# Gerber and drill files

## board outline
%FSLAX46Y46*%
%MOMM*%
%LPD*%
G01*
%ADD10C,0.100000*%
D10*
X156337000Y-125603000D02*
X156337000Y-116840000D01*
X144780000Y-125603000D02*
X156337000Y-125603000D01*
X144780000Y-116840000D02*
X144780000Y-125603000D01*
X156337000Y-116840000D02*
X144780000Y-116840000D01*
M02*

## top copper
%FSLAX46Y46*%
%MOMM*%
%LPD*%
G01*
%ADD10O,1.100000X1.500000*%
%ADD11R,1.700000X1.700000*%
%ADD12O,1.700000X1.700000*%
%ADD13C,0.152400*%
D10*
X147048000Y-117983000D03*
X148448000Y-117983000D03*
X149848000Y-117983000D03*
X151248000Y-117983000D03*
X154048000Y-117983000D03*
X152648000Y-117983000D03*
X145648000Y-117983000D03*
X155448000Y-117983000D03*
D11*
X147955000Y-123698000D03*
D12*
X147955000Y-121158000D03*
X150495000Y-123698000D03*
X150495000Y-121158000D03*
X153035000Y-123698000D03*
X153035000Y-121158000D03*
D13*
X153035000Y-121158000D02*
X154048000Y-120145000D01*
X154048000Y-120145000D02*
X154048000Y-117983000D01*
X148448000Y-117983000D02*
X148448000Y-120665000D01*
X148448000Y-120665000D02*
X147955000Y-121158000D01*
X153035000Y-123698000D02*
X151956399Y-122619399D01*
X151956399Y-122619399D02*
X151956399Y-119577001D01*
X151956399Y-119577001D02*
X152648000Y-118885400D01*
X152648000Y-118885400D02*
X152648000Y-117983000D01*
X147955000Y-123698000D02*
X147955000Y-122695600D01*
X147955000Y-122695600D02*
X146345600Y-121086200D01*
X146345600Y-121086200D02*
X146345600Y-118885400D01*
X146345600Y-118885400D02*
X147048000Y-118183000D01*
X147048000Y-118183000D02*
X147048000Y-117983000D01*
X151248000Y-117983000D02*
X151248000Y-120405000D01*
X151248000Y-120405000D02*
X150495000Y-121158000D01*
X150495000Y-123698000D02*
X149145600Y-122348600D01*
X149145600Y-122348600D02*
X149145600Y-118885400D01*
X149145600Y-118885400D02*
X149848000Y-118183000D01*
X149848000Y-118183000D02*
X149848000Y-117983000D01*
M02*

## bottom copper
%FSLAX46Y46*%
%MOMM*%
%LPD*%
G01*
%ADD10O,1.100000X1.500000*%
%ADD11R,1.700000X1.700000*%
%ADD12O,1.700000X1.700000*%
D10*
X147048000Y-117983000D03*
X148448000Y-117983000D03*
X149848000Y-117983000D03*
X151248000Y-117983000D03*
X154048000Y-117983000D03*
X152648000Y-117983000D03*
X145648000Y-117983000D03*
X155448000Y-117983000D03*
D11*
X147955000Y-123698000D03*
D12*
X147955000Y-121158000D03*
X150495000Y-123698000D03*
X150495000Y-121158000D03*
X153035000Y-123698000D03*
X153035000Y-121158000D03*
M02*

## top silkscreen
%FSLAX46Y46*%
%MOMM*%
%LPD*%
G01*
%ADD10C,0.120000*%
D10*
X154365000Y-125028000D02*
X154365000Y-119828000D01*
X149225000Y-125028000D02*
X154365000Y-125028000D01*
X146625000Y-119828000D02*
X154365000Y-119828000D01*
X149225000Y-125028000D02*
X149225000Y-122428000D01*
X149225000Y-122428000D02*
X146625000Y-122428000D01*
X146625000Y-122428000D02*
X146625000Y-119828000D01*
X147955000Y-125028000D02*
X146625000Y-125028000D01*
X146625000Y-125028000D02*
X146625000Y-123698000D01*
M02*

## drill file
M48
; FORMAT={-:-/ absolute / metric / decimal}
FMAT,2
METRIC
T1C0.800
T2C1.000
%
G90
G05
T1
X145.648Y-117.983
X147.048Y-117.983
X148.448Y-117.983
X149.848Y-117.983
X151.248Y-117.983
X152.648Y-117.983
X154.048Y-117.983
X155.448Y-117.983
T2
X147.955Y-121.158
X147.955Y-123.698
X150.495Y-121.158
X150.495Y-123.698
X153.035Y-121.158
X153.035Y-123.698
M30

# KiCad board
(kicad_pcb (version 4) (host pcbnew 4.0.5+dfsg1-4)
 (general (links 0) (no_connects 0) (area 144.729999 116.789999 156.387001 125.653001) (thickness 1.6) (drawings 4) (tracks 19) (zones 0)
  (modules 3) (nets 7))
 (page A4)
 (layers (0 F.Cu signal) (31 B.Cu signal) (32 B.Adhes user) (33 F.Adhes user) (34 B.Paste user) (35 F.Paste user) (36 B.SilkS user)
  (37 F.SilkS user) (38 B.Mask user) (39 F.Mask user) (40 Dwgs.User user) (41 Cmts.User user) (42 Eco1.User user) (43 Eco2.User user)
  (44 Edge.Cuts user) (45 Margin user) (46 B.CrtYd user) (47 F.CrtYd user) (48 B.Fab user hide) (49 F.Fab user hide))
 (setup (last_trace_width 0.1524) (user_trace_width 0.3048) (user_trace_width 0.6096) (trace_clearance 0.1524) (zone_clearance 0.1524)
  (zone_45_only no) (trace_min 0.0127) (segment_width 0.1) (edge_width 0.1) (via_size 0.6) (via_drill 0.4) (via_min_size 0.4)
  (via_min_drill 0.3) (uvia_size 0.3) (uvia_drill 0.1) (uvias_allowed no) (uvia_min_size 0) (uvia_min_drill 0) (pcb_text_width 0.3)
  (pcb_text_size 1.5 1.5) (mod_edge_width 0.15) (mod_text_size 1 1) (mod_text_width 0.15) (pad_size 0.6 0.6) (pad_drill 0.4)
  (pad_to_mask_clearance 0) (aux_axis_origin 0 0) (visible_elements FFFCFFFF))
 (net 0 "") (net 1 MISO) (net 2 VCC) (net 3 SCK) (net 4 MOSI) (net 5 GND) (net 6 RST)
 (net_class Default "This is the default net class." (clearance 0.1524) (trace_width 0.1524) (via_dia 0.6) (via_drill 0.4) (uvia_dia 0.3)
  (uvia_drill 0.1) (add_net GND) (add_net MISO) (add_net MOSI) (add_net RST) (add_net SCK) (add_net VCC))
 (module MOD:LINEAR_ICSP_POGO (layer F.Cu) (at 150.548 116.583)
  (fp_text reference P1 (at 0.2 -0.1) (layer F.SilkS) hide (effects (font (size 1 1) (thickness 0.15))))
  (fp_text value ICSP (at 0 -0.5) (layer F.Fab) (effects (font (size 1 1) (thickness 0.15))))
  (pad 1 thru_hole oval (at -3.5 1.4) (size 1.1 1.5) (drill 0.8) (layers *.Cu *.Mask) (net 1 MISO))
  (pad 2 thru_hole oval (at -2.1 1.4) (size 1.1 1.5) (drill 0.8) (layers *.Cu *.Mask) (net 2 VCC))
  (pad 3 thru_hole oval (at -0.7 1.4) (size 1.1 1.5) (drill 0.8) (layers *.Cu *.Mask) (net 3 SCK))
  (pad 4 thru_hole oval (at 0.7 1.4) (size 1.1 1.5) (drill 0.8) (layers *.Cu *.Mask) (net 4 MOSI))
  (pad 6 thru_hole oval (at 3.5 1.4) (size 1.1 1.5) (drill 0.8) (layers *.Cu *.Mask) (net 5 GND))
  (pad 5 thru_hole oval (at 2.1 1.4) (size 1.1 1.5) (drill 0.8) (layers *.Cu *.Mask) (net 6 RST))
  (pad NC1 thru_hole oval (at -4.9 1.4) (size 1.1 1.5) (drill 0.8) (layers *.Cu *.Mask))
  (pad NC2 thru_hole oval (at 4.9 1.4) (size 1.1 1.5) (drill 0.8) (layers *.Cu *.Mask)))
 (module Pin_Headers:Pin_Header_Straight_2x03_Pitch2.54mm (layer F.Cu) (at 147.955 123.698 90)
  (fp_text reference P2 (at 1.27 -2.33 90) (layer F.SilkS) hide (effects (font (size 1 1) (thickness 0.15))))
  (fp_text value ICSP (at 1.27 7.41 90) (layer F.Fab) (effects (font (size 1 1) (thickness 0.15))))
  (fp_line (start -1.33 6.41) (end 3.87 6.41) (layer F.SilkS) (width 0.12))
  (fp_line (start -1.33 1.27) (end -1.33 6.41) (layer F.SilkS) (width 0.12))
  (fp_line (start 3.87 -1.33) (end 3.87 6.41) (layer F.SilkS) (width 0.12))
  (fp_line (start -1.33 1.27) (end 1.27 1.27) (layer F.SilkS) (width 0.12))
  (fp_line (start 1.27 1.27) (end 1.27 -1.33) (layer F.SilkS) (width 0.12))
  (fp_line (start 1.27 -1.33) (end 3.87 -1.33) (layer F.SilkS) (width 0.12))
  (fp_line (start -1.33 0) (end -1.33 -1.33) (layer F.SilkS) (width 0.12))
  (fp_line (start -1.33 -1.33) (end 0 -1.33) (layer F.SilkS) (width 0.12))
  (pad 1 thru_hole rect (at 0 0 90) (size 1.7 1.7) (drill 1) (layers *.Cu *.Mask) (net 1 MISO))
  (pad 2 thru_hole oval (at 2.54 0 90) (size 1.7 1.7) (drill 1) (layers *.Cu *.Mask) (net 2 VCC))
  (pad 3 thru_hole oval (at 0 2.54 90) (size 1.7 1.7) (drill 1) (layers *.Cu *.Mask) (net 3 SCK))
  (pad 4 thru_hole oval (at 2.54 2.54 90) (size 1.7 1.7) (drill 1) (layers *.Cu *.Mask) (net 4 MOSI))
  (pad 5 thru_hole oval (at 0 5.08 90) (size 1.7 1.7) (drill 1) (layers *.Cu *.Mask) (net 6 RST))
  (pad 6 thru_hole oval (at 2.54 5.08 90) (size 1.7 1.7) (drill 1) (layers *.Cu *.Mask) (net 5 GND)))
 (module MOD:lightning (layer B.Cu) (at 154.94 122.555)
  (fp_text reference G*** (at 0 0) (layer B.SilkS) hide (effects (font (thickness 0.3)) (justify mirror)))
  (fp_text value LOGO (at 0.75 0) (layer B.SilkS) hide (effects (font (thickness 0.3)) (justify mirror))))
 (gr_line (start 156.337 125.603) (end 156.337 116.84) (layer Edge.Cuts) (width 0.1))
 (gr_line (start 144.78 125.603) (end 156.337 125.603) (layer Edge.Cuts) (width 0.1))
 (gr_line (start 144.78 116.84) (end 144.78 125.603) (layer Edge.Cuts) (width 0.1))
 (gr_line (start 156.337 116.84) (end 144.78 116.84) (layer Edge.Cuts) (width 0.1))
 (segment (start 153.035 121.158) (end 154.048 120.145) (width 0.1524) (layer F.Cu) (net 5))
 (segment (start 154.048 120.145) (end 154.048 117.983) (width 0.1524) (layer F.Cu) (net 5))
 (segment (start 148.448 117.983) (end 148.448 120.665) (width 0.1524) (layer F.Cu) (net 2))
 (segment (start 148.448 120.665) (end 147.955 121.158) (width 0.1524) (layer F.Cu) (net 2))
 (segment (start 153.035 123.698) (end 151.956399 122.619399) (width 0.1524) (layer F.Cu) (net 6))
 (segment (start 151.956399 122.619399) (end 151.956399 119.577001) (width 0.1524) (layer F.Cu) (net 6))
 (segment (start 151.956399 119.577001) (end 152.648 118.8854) (width 0.1524) (layer F.Cu) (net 6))
 (segment (start 152.648 118.8854) (end 152.648 117.983) (width 0.1524) (layer F.Cu) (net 6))
 (segment (start 147.955 123.698) (end 147.955 122.6956) (width 0.1524) (layer F.Cu) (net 1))
 (segment (start 147.955 122.6956) (end 146.3456 121.0862) (width 0.1524) (layer F.Cu) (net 1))
 (segment (start 146.3456 121.0862) (end 146.3456 118.8854) (width 0.1524) (layer F.Cu) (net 1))
 (segment (start 146.3456 118.8854) (end 147.048 118.183) (width 0.1524) (layer F.Cu) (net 1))
 (segment (start 147.048 118.183) (end 147.048 117.983) (width 0.1524) (layer F.Cu) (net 1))
 (segment (start 151.248 117.983) (end 151.248 120.405) (width 0.1524) (layer F.Cu) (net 4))
 (segment (start 151.248 120.405) (end 150.495 121.158) (width 0.1524) (layer F.Cu) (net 4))
 (segment (start 150.495 123.698) (end 149.1456 122.3486) (width 0.1524) (layer F.Cu) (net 3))
 (segment (start 149.1456 122.3486) (end 149.1456 118.8854) (width 0.1524) (layer F.Cu) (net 3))
 (segment (start 149.1456 118.8854) (end 149.848 118.183) (width 0.1524) (layer F.Cu) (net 3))
 (segment (start 149.848 118.183) (end 149.848 117.983) (width 0.1524) (layer F.Cu) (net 3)))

